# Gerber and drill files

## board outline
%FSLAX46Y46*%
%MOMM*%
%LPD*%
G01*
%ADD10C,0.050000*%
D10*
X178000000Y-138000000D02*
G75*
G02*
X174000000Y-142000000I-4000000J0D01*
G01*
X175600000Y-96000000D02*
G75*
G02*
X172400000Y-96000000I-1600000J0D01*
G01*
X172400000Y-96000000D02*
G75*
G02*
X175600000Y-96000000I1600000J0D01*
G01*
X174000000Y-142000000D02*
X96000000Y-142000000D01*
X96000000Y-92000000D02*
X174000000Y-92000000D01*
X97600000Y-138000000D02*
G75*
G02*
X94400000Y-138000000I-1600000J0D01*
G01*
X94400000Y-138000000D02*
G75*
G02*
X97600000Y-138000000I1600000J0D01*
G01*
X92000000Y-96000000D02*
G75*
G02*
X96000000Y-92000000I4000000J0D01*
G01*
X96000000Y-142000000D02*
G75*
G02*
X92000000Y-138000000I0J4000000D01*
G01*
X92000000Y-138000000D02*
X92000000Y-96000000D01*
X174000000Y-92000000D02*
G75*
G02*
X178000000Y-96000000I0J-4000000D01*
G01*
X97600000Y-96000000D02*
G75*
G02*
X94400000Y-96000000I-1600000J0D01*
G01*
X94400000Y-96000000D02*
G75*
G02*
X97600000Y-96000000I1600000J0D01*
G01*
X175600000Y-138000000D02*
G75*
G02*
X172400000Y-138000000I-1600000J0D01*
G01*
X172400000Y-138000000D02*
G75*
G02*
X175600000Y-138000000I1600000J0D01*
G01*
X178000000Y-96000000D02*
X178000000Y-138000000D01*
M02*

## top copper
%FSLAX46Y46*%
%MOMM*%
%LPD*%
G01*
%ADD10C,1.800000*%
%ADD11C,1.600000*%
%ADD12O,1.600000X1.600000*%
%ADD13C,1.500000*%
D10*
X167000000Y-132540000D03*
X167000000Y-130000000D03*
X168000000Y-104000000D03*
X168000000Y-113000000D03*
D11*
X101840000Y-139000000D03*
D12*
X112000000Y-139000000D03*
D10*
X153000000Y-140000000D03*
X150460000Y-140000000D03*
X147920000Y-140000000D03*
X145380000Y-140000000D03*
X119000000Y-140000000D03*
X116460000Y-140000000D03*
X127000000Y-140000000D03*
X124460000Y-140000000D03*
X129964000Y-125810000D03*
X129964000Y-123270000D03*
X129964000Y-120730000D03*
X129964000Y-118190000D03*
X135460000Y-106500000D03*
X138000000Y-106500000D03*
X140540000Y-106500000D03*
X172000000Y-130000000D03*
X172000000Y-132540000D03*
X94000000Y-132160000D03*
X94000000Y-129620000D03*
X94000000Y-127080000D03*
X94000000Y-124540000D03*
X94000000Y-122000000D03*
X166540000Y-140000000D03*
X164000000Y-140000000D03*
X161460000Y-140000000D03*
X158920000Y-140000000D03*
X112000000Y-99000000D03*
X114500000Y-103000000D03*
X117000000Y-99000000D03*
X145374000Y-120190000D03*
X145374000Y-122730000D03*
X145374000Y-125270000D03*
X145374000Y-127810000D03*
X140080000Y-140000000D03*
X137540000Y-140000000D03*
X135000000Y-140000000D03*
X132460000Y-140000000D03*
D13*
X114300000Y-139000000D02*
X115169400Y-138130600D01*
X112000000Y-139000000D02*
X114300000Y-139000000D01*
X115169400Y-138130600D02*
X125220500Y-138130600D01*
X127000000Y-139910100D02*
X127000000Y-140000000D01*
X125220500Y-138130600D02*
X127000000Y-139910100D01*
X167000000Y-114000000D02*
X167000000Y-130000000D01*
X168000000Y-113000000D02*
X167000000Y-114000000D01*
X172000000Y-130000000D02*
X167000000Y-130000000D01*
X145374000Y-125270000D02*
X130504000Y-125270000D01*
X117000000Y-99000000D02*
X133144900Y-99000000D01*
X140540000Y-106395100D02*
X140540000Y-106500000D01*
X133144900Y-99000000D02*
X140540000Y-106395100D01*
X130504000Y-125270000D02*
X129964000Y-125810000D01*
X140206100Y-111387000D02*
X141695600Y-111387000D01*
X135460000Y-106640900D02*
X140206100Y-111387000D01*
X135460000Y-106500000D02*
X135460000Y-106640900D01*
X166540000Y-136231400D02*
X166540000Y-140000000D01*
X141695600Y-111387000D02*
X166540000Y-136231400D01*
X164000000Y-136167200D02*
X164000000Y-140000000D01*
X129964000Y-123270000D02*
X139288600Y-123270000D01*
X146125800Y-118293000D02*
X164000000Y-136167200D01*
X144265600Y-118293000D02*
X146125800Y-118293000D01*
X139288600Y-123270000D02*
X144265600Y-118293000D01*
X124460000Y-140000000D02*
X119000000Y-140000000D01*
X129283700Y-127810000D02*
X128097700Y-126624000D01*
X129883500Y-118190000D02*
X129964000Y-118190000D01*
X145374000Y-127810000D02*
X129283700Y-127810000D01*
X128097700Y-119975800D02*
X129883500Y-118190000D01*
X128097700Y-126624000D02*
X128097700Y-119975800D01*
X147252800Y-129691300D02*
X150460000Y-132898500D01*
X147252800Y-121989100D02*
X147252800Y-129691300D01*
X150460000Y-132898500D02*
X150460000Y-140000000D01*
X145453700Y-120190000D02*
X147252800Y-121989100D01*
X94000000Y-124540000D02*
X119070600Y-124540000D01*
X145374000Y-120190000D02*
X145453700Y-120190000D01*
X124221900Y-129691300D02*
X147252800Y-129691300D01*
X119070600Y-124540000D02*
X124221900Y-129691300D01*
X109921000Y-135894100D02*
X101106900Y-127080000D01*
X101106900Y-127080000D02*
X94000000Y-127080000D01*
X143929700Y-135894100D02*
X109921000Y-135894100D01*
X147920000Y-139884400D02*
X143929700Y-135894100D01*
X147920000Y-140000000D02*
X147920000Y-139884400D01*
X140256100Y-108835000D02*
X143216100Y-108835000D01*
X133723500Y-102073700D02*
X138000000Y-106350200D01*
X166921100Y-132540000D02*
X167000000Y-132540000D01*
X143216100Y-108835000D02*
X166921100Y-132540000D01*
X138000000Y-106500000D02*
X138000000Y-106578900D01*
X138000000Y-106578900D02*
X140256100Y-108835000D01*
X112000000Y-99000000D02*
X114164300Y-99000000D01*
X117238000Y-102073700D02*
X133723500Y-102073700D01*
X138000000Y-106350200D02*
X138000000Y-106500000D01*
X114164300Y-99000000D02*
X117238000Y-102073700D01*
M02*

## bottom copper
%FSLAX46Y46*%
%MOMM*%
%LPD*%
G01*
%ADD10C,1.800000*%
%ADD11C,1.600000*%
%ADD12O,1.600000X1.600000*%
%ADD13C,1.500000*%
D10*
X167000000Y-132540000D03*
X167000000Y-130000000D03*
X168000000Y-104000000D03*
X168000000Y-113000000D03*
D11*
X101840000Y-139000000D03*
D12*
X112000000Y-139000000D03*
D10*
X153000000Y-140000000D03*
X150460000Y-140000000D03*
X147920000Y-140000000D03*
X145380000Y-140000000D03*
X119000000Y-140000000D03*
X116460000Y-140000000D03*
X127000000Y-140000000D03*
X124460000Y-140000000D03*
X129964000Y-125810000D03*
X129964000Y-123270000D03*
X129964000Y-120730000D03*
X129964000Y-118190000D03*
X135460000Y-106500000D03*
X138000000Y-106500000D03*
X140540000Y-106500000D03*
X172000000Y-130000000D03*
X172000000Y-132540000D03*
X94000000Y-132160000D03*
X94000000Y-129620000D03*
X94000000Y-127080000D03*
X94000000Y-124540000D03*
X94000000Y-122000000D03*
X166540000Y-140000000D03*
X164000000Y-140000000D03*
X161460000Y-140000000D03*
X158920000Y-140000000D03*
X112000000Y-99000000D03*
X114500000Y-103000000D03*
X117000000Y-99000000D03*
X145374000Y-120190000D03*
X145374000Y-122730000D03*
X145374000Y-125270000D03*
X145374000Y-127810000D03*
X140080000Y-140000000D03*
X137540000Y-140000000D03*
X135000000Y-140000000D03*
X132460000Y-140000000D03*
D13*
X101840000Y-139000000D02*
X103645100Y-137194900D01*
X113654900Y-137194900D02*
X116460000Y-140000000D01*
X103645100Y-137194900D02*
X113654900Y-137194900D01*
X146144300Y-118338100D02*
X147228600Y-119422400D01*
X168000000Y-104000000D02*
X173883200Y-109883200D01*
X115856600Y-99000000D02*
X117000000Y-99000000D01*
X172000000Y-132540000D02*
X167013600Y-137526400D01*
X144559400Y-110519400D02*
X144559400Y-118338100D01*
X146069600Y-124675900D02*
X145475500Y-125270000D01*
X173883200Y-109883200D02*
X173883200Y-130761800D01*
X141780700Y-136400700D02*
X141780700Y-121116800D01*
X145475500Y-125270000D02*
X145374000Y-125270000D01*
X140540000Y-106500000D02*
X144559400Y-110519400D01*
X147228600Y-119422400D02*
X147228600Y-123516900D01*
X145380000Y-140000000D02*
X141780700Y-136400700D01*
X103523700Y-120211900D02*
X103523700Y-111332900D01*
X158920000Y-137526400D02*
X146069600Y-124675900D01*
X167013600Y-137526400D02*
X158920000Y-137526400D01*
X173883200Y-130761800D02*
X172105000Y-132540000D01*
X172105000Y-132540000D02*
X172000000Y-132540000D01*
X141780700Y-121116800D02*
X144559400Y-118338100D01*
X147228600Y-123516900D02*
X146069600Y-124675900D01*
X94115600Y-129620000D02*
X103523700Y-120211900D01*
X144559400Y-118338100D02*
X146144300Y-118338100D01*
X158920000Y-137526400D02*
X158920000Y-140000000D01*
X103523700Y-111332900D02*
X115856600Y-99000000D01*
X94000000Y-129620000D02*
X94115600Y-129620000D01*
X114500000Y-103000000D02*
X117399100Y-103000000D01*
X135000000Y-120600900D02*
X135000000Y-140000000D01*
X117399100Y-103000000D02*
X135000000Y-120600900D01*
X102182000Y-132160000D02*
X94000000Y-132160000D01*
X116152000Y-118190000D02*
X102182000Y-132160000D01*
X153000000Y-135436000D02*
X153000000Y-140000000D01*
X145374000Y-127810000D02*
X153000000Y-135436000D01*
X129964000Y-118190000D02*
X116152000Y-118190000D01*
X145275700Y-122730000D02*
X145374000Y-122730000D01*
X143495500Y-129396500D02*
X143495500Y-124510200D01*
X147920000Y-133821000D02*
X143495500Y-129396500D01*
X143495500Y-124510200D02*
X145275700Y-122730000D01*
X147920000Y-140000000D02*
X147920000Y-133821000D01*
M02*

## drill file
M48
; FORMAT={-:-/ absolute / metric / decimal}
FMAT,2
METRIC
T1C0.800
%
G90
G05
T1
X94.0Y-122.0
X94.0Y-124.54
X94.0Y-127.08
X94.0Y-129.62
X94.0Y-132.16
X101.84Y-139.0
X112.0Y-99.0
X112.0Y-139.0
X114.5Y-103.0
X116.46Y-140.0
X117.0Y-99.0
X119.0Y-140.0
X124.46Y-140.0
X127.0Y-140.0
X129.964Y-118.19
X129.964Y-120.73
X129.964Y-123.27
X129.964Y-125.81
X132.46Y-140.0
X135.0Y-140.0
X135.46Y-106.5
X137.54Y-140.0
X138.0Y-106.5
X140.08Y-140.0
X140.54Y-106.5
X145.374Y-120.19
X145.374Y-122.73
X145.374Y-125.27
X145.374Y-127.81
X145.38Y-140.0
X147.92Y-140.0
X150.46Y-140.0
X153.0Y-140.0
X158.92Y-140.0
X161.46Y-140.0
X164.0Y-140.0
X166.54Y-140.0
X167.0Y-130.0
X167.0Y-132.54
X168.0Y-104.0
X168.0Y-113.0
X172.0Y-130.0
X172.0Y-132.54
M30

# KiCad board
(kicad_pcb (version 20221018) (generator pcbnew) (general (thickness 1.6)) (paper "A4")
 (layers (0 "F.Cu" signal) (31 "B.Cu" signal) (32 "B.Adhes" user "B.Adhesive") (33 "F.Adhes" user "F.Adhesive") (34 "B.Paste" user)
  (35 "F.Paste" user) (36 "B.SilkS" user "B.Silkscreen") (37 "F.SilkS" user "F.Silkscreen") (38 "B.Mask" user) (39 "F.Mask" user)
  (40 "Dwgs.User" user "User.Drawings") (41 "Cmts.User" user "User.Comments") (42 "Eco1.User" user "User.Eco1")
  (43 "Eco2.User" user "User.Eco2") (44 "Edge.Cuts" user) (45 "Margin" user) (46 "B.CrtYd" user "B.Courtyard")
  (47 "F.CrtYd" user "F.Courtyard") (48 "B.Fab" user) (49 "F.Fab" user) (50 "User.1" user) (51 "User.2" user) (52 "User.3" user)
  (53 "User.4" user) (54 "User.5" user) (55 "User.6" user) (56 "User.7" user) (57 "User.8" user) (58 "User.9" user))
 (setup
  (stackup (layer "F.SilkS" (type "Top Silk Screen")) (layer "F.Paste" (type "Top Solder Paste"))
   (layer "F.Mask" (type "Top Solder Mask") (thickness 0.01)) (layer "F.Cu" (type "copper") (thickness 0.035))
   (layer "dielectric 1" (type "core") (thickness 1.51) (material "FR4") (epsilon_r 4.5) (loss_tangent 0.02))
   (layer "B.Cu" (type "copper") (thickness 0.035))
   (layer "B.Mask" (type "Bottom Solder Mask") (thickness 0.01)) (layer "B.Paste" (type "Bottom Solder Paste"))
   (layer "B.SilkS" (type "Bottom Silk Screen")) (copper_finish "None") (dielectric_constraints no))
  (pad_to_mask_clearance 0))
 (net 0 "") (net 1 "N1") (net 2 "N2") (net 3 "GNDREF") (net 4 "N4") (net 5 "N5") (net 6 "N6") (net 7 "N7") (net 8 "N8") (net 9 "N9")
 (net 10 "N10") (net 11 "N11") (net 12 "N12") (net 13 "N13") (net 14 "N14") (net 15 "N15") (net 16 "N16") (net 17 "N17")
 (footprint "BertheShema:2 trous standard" (layer "F.Cu") (at 167 132.54)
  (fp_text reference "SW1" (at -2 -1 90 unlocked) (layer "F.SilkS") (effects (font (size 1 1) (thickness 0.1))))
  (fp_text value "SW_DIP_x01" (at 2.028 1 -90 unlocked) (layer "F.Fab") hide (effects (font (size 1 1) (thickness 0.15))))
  (pad "1" thru_hole circle (at 0 0) (size 1.8 1.8) (drill 0.8) (layers "*.Cu" "*.Mask") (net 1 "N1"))
  (pad "2" thru_hole circle (at 0 -2.54) (size 1.8 1.8) (drill 0.8) (layers "*.Cu" "*.Mask") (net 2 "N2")))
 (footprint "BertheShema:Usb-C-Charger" (layer "F.Cu") (at 175 107 -90)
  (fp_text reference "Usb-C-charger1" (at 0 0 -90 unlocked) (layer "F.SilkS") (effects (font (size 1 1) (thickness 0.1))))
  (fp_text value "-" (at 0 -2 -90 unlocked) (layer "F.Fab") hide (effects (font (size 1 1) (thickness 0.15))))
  (pad "1" thru_hole circle (at -3 7 270) (size 1.8 1.8) (drill 0.8) (layers "*.Cu" "*.Mask") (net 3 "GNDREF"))
  (pad "2" thru_hole circle (at 6 7 270) (size 1.8 1.8) (drill 0.8) (layers "*.Cu" "*.Mask") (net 2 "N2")))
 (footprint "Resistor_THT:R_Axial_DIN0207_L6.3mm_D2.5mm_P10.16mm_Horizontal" (layer "F.Cu") (at 101.84 139)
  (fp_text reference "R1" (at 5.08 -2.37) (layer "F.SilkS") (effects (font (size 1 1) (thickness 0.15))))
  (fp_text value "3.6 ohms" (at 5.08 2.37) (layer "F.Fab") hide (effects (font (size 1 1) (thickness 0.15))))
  (pad "1" thru_hole circle (at 0 0) (size 1.6 1.6) (drill 0.8) (layers "*.Cu" "*.Mask") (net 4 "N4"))
  (pad "2" thru_hole oval (at 10.16 0) (size 1.6 1.6) (drill 0.8) (layers "*.Cu" "*.Mask") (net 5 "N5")))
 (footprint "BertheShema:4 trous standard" (layer "F.Cu") (at 150.46 140 90)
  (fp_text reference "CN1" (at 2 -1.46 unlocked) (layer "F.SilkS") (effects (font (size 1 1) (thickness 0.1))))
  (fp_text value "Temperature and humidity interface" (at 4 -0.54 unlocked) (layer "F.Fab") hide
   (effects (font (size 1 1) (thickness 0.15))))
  (pad "1" thru_hole circle (at 0 2.54 90) (size 1.8 1.8) (drill 0.8) (layers "*.Cu" "*.Mask") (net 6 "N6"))
  (pad "2" thru_hole circle (at 0 0 90) (size 1.8 1.8) (drill 0.8) (layers "*.Cu" "*.Mask") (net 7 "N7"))
  (pad "3" thru_hole circle (at 0 -2.54 90) (size 1.8 1.8) (drill 0.8) (layers "*.Cu" "*.Mask") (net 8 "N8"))
  (pad "4" thru_hole circle (at 0 -5.08 90) (size 1.8 1.8) (drill 0.8) (layers "*.Cu" "*.Mask") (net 3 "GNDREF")))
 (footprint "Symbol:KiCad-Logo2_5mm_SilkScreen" (layer "F.Cu") (at 152 111)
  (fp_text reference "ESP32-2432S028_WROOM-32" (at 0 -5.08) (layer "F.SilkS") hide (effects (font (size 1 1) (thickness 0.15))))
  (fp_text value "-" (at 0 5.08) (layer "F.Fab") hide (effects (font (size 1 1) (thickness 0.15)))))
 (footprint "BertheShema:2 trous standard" (layer "F.Cu") (at 119 140 90)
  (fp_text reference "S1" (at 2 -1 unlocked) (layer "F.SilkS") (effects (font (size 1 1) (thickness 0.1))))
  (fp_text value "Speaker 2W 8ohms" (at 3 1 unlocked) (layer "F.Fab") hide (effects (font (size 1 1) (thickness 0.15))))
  (pad "1" thru_hole circle (at 0 0 90) (size 1.8 1.8) (drill 0.8) (layers "*.Cu" "*.Mask") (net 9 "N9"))
  (pad "2" thru_hole circle (at 0 -2.54 90) (size 1.8 1.8) (drill 0.8) (layers "*.Cu" "*.Mask") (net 4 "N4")))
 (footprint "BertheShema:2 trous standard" (layer "F.Cu") (at 127 140 90)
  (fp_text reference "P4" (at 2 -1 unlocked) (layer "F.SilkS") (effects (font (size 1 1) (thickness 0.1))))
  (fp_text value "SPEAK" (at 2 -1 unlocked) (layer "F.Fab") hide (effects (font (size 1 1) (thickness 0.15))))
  (pad "1" thru_hole circle (at 0 0 90) (size 1.8 1.8) (drill 0.8) (layers "*.Cu" "*.Mask") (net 5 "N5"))
  (pad "2" thru_hole circle (at 0 -2.54 90) (size 1.8 1.8) (drill 0.8) (layers "*.Cu" "*.Mask") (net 9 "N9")))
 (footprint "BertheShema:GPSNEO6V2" (layer "F.Cu") (at 128.44 122 90)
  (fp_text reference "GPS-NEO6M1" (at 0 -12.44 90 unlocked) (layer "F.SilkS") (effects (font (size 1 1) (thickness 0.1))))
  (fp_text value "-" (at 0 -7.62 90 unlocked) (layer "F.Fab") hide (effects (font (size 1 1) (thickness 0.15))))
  (pad "1" thru_hole circle (at -3.81 1.524 90) (size 1.8 1.8) (drill 0.8) (layers "*.Cu" "*.Mask") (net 3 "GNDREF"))
  (pad "2" thru_hole circle (at -1.27 1.524 90) (size 1.8 1.8) (drill 0.8) (layers "*.Cu" "*.Mask") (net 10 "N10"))
  (pad "3" thru_hole circle (at 1.27 1.524 90) (size 1.8 1.8) (drill 0.8) (layers "*.Cu" "*.Mask") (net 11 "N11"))
  (pad "4" thru_hole circle (at 3.81 1.524 90) (size 1.8 1.8) (drill 0.8) (layers "*.Cu" "*.Mask") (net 6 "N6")))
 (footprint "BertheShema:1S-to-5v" (layer "F.Cu") (at 138 102.5)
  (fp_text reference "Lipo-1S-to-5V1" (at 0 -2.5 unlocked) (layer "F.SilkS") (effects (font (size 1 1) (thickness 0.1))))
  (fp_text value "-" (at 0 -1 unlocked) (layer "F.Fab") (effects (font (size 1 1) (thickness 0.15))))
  (pad "1" thru_hole circle (at -2.54 4) (size 1.8 1.8) (drill 0.8) (layers "*.Cu" "*.Mask") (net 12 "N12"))
  (pad "2" thru_hole circle (at 0 4) (size 1.8 1.8) (drill 0.8) (layers "*.Cu" "*.Mask") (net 1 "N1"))
  (pad "3" thru_hole circle (at 2.54 4) (size 1.8 1.8) (drill 0.8) (layers "*.Cu" "*.Mask") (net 3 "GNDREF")))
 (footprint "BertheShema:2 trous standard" (layer "F.Cu") (at 172 130 180)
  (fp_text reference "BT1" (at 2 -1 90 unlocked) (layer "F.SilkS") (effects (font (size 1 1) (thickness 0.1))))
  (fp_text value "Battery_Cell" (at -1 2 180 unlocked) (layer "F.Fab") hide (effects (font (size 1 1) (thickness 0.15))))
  (pad "1" thru_hole circle (at 0 0 180) (size 1.8 1.8) (drill 0.8) (layers "*.Cu" "*.Mask") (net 2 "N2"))
  (pad "2" thru_hole circle (at 0 -2.54 180) (size 1.8 1.8) (drill 0.8) (layers "*.Cu" "*.Mask") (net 3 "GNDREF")))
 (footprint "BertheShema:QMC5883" (layer "F.Cu") (at 88.92 127.08 90)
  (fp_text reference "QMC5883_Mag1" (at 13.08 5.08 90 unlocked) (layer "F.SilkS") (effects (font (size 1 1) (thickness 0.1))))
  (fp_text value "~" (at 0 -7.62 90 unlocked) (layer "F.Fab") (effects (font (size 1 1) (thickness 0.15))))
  (pad "1" thru_hole circle (at -5.08 5.08 90) (size 1.8 1.8) (drill 0.8) (layers "*.Cu" "*.Mask") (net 6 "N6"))
  (pad "2" thru_hole circle (at -2.54 5.08 90) (size 1.8 1.8) (drill 0.8) (layers "*.Cu" "*.Mask") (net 3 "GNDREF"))
  (pad "3" thru_hole circle (at 0 5.08 90) (size 1.8 1.8) (drill 0.8) (layers "*.Cu" "*.Mask") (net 8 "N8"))
  (pad "4" thru_hole circle (at 2.54 5.08 90) (size 1.8 1.8) (drill 0.8) (layers "*.Cu" "*.Mask") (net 7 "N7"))
  (pad "5" thru_hole circle (at 5.08 5.08 90) (size 1.8 1.8) (drill 0.8) (layers "*.Cu" "*.Mask")))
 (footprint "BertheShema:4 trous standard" (layer "F.Cu") (at 164 140 90)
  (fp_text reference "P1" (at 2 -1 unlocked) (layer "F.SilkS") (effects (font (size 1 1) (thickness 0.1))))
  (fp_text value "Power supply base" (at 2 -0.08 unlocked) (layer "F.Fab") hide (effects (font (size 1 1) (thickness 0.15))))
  (pad "1" thru_hole circle (at 0 2.54 90) (size 1.8 1.8) (drill 0.8) (layers "*.Cu" "*.Mask") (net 12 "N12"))
  (pad "2" thru_hole circle (at 0 0 90) (size 1.8 1.8) (drill 0.8) (layers "*.Cu" "*.Mask") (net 10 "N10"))
  (pad "3" thru_hole circle (at 0 -2.54 90) (size 1.8 1.8) (drill 0.8) (layers "*.Cu" "*.Mask") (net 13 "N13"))
  (pad "4" thru_hole circle (at 0 -5.08 90) (size 1.8 1.8) (drill 0.8) (layers "*.Cu" "*.Mask") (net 3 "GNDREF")))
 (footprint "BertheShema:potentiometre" (layer "F.Cu") (at 114.5 99.5)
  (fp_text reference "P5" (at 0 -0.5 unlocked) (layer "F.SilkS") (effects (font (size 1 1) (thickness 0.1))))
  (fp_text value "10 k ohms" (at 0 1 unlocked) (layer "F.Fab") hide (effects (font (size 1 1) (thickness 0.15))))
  (pad "1" thru_hole circle (at -2.5 -0.5) (size 1.8 1.8) (drill 0.8) (layers "*.Cu" "*.Mask") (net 1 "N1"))
  (pad "2" thru_hole circle (at 0 3.5) (size 1.8 1.8) (drill 0.8) (layers "*.Cu" "*.Mask") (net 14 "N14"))
  (pad "3" thru_hole circle (at 2.5 -0.5) (size 1.8 1.8) (drill 0.8) (layers "*.Cu" "*.Mask") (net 3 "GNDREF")))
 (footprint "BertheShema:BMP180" (layer "F.Cu") (at 146.898 124 -90)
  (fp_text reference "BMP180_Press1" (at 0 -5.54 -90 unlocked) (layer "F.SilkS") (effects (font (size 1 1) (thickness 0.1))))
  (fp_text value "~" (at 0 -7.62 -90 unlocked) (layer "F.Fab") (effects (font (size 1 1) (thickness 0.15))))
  (pad "1" thru_hole circle (at -3.81 1.524 270) (size 1.8 1.8) (drill 0.8) (layers "*.Cu" "*.Mask") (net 7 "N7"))
  (pad "2" thru_hole circle (at -1.27 1.524 270) (size 1.8 1.8) (drill 0.8) (layers "*.Cu" "*.Mask") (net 8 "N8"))
  (pad "3" thru_hole circle (at 1.27 1.524 270) (size 1.8 1.8) (drill 0.8) (layers "*.Cu" "*.Mask") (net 3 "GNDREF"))
  (pad "4" thru_hole circle (at 3.81 1.524 270) (size 1.8 1.8) (drill 0.8) (layers "*.Cu" "*.Mask") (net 6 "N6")))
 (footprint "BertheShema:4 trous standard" (layer "F.Cu") (at 137.54 140 90)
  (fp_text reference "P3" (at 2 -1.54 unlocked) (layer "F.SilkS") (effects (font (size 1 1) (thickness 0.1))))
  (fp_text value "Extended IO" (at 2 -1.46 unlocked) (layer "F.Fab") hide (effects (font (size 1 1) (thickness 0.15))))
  (pad "1" thru_hole circle (at 0 2.54 90) (size 1.8 1.8) (drill 0.8) (layers "*.Cu" "*.Mask") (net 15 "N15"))
  (pad "2" thru_hole circle (at 0 0 90) (size 1.8 1.8) (drill 0.8) (layers "*.Cu" "*.Mask") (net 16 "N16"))
  (pad "3" thru_hole circle (at 0 -2.54 90) (size 1.8 1.8) (drill 0.8) (layers "*.Cu" "*.Mask") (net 14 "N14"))
  (pad "4" thru_hole circle (at 0 -5.08 90) (size 1.8 1.8) (drill 0.8) (layers "*.Cu" "*.Mask") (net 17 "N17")))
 (gr_arc (start 178 138) (mid 176.828427 140.828427) (end 174 142) (stroke (width 0.05) (type default)) (layer "Edge.Cuts"))
 (gr_circle (center 174 96) (end 175.6 96) (stroke (width 0.05) (type default)) (fill none) (layer "Edge.Cuts"))
 (gr_line (start 174 142) (end 96 142) (stroke (width 0.05) (type default)) (layer "Edge.Cuts"))
 (gr_line (start 96 92) (end 174 92) (stroke (width 0.05) (type default)) (layer "Edge.Cuts"))
 (gr_circle (center 96 138) (end 97.6 138) (stroke (width 0.05) (type default)) (fill none) (layer "Edge.Cuts"))
 (gr_arc (start 92 96) (mid 93.171573 93.171573) (end 96 92) (stroke (width 0.05) (type default)) (layer "Edge.Cuts"))
 (gr_arc (start 96 142) (mid 93.171573 140.828427) (end 92 138) (stroke (width 0.05) (type default)) (layer "Edge.Cuts"))
 (gr_line (start 92 138) (end 92 96) (stroke (width 0.05) (type default)) (layer "Edge.Cuts"))
 (gr_arc (start 174 92) (mid 176.828427 93.171573) (end 178 96) (stroke (width 0.05) (type default)) (layer "Edge.Cuts"))
 (gr_circle (center 96 96) (end 97.6 96) (stroke (width 0.05) (type default)) (fill none) (layer "Edge.Cuts"))
 (gr_circle (center 174 138) (end 175.6 138) (stroke (width 0.05) (type default)) (fill none) (layer "Edge.Cuts"))
 (gr_line (start 178 96) (end 178 138) (stroke (width 0.05) (type default)) (layer "Edge.Cuts"))
 (segment (start 101.84 139) (end 103.6451 137.1949) (width 1.5) (layer "B.Cu") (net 4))
 (segment (start 113.6549 137.1949) (end 116.46 140) (width 1.5) (layer "B.Cu") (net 4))
 (segment (start 103.6451 137.1949) (end 113.6549 137.1949) (width 1.5) (layer "B.Cu") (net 4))
 (segment (start 114.3 139) (end 115.1694 138.1306) (width 1.5) (layer "F.Cu") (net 5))
 (segment (start 112 139) (end 114.3 139) (width 1.5) (layer "F.Cu") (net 5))
 (segment (start 115.1694 138.1306) (end 125.2205 138.1306) (width 1.5) (layer "F.Cu") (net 5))
 (segment (start 127 139.9101) (end 127 140) (width 1.5) (layer "F.Cu") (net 5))
 (segment (start 125.2205 138.1306) (end 127 139.9101) (width 1.5) (layer "F.Cu") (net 5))
 (segment (start 167 114) (end 167 130) (width 1.5) (layer "F.Cu") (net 2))
 (segment (start 168 113) (end 167 114) (width 1.5) (layer "F.Cu") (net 2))
 (segment (start 172 130) (end 167 130) (width 1.5) (layer "F.Cu") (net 2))
 (segment (start 145.374 125.27) (end 130.504 125.27) (width 1.5) (layer "F.Cu") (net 3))
 (segment (start 117 99) (end 133.1449 99) (width 1.5) (layer "F.Cu") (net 3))
 (segment (start 140.54 106.3951) (end 140.54 106.5) (width 1.5) (layer "F.Cu") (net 3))
 (segment (start 133.1449 99) (end 140.54 106.3951) (width 1.5) (layer "F.Cu") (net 3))
 (segment (start 130.504 125.27) (end 129.964 125.81) (width 1.5) (layer "F.Cu") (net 3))
 (segment (start 146.1443 118.3381) (end 147.2286 119.4224) (width 1.5) (layer "B.Cu") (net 3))
 (segment (start 168 104) (end 173.8832 109.8832) (width 1.5) (layer "B.Cu") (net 3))
 (segment (start 115.8566 99) (end 117 99) (width 1.5) (layer "B.Cu") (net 3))
 (segment (start 172 132.54) (end 167.0136 137.5264) (width 1.5) (layer "B.Cu") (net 3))
 (segment (start 144.5594 110.5194) (end 144.5594 118.3381) (width 1.5) (layer "B.Cu") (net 3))
 (segment (start 146.0696 124.6759) (end 145.4755 125.27) (width 1.5) (layer "B.Cu") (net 3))
 (segment (start 173.8832 109.8832) (end 173.8832 130.7618) (width 1.5) (layer "B.Cu") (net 3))
 (segment (start 141.7807 136.4007) (end 141.7807 121.1168) (width 1.5) (layer "B.Cu") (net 3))
 (segment (start 145.4755 125.27) (end 145.374 125.27) (width 1.5) (layer "B.Cu") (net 3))
 (segment (start 140.54 106.5) (end 144.5594 110.5194) (width 1.5) (layer "B.Cu") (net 3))
 (segment (start 147.2286 119.4224) (end 147.2286 123.5169) (width 1.5) (layer "B.Cu") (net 3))
 (segment (start 145.38 140) (end 141.7807 136.4007) (width 1.5) (layer "B.Cu") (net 3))
 (segment (start 103.5237 120.2119) (end 103.5237 111.3329) (width 1.5) (layer "B.Cu") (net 3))
 (segment (start 158.92 137.5264) (end 146.0696 124.6759) (width 1.5) (layer "B.Cu") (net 3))
 (segment (start 167.0136 137.5264) (end 158.92 137.5264) (width 1.5) (layer "B.Cu") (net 3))
 (segment (start 173.8832 130.7618) (end 172.105 132.54) (width 1.5) (layer "B.Cu") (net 3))
 (segment (start 172.105 132.54) (end 172 132.54) (width 1.5) (layer "B.Cu") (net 3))
 (segment (start 141.7807 121.1168) (end 144.5594 118.3381) (width 1.5) (layer "B.Cu") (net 3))
 (segment (start 147.2286 123.5169) (end 146.0696 124.6759) (width 1.5) (layer "B.Cu") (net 3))
 (segment (start 94.1156 129.62) (end 103.5237 120.2119) (width 1.5) (layer "B.Cu") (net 3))
 (segment (start 144.5594 118.3381) (end 146.1443 118.3381) (width 1.5) (layer "B.Cu") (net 3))
 (segment (start 158.92 137.5264) (end 158.92 140) (width 1.5) (layer "B.Cu") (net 3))
 (segment (start 103.5237 111.3329) (end 115.8566 99) (width 1.5) (layer "B.Cu") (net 3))
 (segment (start 94 129.62) (end 94.1156 129.62) (width 1.5) (layer "B.Cu") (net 3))
 (segment (start 140.2061 111.387) (end 141.6956 111.387) (width 1.5) (layer "F.Cu") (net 12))
 (segment (start 135.46 106.6409) (end 140.2061 111.387) (width 1.5) (layer "F.Cu") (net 12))
 (segment (start 135.46 106.5) (end 135.46 106.6409) (width 1.5) (layer "F.Cu") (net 12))
 (segment (start 166.54 136.2314) (end 166.54 140) (width 1.5) (layer "F.Cu") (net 12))
 (segment (start 141.6956 111.387) (end 166.54 136.2314) (width 1.5) (layer "F.Cu") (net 12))
 (segment (start 164 136.1672) (end 164 140) (width 1.5) (layer "F.Cu") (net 10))
 (segment (start 129.964 123.27) (end 139.2886 123.27) (width 1.5) (layer "F.Cu") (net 10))
 (segment (start 146.1258 118.293) (end 164 136.1672) (width 1.5) (layer "F.Cu") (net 10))
 (segment (start 144.2656 118.293) (end 146.1258 118.293) (width 1.5) (layer "F.Cu") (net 10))
 (segment (start 139.2886 123.27) (end 144.2656 118.293) (width 1.5) (layer "F.Cu") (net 10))
 (segment (start 114.5 103) (end 117.3991 103) (width 1.5) (layer "B.Cu") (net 14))
 (segment (start 135 120.6009) (end 135 140) (width 1.5) (layer "B.Cu") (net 14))
 (segment (start 117.3991 103) (end 135 120.6009) (width 1.5) (layer "B.Cu") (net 14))
 (segment (start 124.46 140) (end 119 140) (width 1.5) (layer "F.Cu") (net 9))
 (segment (start 129.2837 127.81) (end 128.0977 126.624) (width 1.5) (layer "F.Cu") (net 6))
 (segment (start 129.8835 118.19) (end 129.964 118.19) (width 1.5) (layer "F.Cu") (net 6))
 (segment (start 145.374 127.81) (end 129.2837 127.81) (width 1.5) (layer "F.Cu") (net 6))
 (segment (start 128.0977 119.9758) (end 129.8835 118.19) (width 1.5) (layer "F.Cu") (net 6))
 (segment (start 128.0977 126.624) (end 128.0977 119.9758) (width 1.5) (layer "F.Cu") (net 6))
 (segment (start 102.182 132.16) (end 94 132.16) (width 1.5) (layer "B.Cu") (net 6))
 (segment (start 116.152 118.19) (end 102.182 132.16) (width 1.5) (layer "B.Cu") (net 6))
 (segment (start 153 135.436) (end 153 140) (width 1.5) (layer "B.Cu") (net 6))
 (segment (start 145.374 127.81) (end 153 135.436) (width 1.5) (layer "B.Cu") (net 6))
 (segment (start 129.964 118.19) (end 116.152 118.19) (width 1.5) (layer "B.Cu") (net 6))
 (segment (start 147.2528 129.6913) (end 150.46 132.8985) (width 1.5) (layer "F.Cu") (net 7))
 (segment (start 147.2528 121.9891) (end 147.2528 129.6913) (width 1.5) (layer "F.Cu") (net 7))
 (segment (start 150.46 132.8985) (end 150.46 140) (width 1.5) (layer "F.Cu") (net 7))
 (segment (start 145.4537 120.19) (end 147.2528 121.9891) (width 1.5) (layer "F.Cu") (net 7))
 (segment (start 94 124.54) (end 119.0706 124.54) (width 1.5) (layer "F.Cu") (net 7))
 (segment (start 145.374 120.19) (end 145.4537 120.19) (width 1.5) (layer "F.Cu") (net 7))
 (segment (start 124.2219 129.6913) (end 147.2528 129.6913) (width 1.5) (layer "F.Cu") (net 7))
 (segment (start 119.0706 124.54) (end 124.2219 129.6913) (width 1.5) (layer "F.Cu") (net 7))
 (segment (start 109.921 135.8941) (end 101.1069 127.08) (width 1.5) (layer "F.Cu") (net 8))
 (segment (start 101.1069 127.08) (end 94 127.08) (width 1.5) (layer "F.Cu") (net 8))
 (segment (start 143.9297 135.8941) (end 109.921 135.8941) (width 1.5) (layer "F.Cu") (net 8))
 (segment (start 147.92 139.8844) (end 143.9297 135.8941) (width 1.5) (layer "F.Cu") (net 8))
 (segment (start 147.92 140) (end 147.92 139.8844) (width 1.5) (layer "F.Cu") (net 8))
 (segment (start 145.2757 122.73) (end 145.374 122.73) (width 1.5) (layer "B.Cu") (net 8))
 (segment (start 143.4955 129.3965) (end 143.4955 124.5102) (width 1.5) (layer "B.Cu") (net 8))
 (segment (start 147.92 133.821) (end 143.4955 129.3965) (width 1.5) (layer "B.Cu") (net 8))
 (segment (start 143.4955 124.5102) (end 145.2757 122.73) (width 1.5) (layer "B.Cu") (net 8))
 (segment (start 147.92 140) (end 147.92 133.821) (width 1.5) (layer "B.Cu") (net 8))
 (segment (start 140.2561 108.835) (end 143.2161 108.835) (width 1.5) (layer "F.Cu") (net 1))
 (segment (start 133.7235 102.0737) (end 138 106.3502) (width 1.5) (layer "F.Cu") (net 1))
 (segment (start 166.9211 132.54) (end 167 132.54) (width 1.5) (layer "F.Cu") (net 1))
 (segment (start 143.2161 108.835) (end 166.9211 132.54) (width 1.5) (layer "F.Cu") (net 1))
 (segment (start 138 106.5) (end 138 106.5789) (width 1.5) (layer "F.Cu") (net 1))
 (segment (start 138 106.5789) (end 140.2561 108.835) (width 1.5) (layer "F.Cu") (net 1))
 (segment (start 112 99) (end 114.1643 99) (width 1.5) (layer "F.Cu") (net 1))
 (segment (start 117.238 102.0737) (end 133.7235 102.0737) (width 1.5) (layer "F.Cu") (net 1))
 (segment (start 138 106.3502) (end 138 106.5) (width 1.5) (layer "F.Cu") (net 1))
 (segment (start 114.1643 99) (end 117.238 102.0737) (width 1.5) (layer "F.Cu") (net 1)))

